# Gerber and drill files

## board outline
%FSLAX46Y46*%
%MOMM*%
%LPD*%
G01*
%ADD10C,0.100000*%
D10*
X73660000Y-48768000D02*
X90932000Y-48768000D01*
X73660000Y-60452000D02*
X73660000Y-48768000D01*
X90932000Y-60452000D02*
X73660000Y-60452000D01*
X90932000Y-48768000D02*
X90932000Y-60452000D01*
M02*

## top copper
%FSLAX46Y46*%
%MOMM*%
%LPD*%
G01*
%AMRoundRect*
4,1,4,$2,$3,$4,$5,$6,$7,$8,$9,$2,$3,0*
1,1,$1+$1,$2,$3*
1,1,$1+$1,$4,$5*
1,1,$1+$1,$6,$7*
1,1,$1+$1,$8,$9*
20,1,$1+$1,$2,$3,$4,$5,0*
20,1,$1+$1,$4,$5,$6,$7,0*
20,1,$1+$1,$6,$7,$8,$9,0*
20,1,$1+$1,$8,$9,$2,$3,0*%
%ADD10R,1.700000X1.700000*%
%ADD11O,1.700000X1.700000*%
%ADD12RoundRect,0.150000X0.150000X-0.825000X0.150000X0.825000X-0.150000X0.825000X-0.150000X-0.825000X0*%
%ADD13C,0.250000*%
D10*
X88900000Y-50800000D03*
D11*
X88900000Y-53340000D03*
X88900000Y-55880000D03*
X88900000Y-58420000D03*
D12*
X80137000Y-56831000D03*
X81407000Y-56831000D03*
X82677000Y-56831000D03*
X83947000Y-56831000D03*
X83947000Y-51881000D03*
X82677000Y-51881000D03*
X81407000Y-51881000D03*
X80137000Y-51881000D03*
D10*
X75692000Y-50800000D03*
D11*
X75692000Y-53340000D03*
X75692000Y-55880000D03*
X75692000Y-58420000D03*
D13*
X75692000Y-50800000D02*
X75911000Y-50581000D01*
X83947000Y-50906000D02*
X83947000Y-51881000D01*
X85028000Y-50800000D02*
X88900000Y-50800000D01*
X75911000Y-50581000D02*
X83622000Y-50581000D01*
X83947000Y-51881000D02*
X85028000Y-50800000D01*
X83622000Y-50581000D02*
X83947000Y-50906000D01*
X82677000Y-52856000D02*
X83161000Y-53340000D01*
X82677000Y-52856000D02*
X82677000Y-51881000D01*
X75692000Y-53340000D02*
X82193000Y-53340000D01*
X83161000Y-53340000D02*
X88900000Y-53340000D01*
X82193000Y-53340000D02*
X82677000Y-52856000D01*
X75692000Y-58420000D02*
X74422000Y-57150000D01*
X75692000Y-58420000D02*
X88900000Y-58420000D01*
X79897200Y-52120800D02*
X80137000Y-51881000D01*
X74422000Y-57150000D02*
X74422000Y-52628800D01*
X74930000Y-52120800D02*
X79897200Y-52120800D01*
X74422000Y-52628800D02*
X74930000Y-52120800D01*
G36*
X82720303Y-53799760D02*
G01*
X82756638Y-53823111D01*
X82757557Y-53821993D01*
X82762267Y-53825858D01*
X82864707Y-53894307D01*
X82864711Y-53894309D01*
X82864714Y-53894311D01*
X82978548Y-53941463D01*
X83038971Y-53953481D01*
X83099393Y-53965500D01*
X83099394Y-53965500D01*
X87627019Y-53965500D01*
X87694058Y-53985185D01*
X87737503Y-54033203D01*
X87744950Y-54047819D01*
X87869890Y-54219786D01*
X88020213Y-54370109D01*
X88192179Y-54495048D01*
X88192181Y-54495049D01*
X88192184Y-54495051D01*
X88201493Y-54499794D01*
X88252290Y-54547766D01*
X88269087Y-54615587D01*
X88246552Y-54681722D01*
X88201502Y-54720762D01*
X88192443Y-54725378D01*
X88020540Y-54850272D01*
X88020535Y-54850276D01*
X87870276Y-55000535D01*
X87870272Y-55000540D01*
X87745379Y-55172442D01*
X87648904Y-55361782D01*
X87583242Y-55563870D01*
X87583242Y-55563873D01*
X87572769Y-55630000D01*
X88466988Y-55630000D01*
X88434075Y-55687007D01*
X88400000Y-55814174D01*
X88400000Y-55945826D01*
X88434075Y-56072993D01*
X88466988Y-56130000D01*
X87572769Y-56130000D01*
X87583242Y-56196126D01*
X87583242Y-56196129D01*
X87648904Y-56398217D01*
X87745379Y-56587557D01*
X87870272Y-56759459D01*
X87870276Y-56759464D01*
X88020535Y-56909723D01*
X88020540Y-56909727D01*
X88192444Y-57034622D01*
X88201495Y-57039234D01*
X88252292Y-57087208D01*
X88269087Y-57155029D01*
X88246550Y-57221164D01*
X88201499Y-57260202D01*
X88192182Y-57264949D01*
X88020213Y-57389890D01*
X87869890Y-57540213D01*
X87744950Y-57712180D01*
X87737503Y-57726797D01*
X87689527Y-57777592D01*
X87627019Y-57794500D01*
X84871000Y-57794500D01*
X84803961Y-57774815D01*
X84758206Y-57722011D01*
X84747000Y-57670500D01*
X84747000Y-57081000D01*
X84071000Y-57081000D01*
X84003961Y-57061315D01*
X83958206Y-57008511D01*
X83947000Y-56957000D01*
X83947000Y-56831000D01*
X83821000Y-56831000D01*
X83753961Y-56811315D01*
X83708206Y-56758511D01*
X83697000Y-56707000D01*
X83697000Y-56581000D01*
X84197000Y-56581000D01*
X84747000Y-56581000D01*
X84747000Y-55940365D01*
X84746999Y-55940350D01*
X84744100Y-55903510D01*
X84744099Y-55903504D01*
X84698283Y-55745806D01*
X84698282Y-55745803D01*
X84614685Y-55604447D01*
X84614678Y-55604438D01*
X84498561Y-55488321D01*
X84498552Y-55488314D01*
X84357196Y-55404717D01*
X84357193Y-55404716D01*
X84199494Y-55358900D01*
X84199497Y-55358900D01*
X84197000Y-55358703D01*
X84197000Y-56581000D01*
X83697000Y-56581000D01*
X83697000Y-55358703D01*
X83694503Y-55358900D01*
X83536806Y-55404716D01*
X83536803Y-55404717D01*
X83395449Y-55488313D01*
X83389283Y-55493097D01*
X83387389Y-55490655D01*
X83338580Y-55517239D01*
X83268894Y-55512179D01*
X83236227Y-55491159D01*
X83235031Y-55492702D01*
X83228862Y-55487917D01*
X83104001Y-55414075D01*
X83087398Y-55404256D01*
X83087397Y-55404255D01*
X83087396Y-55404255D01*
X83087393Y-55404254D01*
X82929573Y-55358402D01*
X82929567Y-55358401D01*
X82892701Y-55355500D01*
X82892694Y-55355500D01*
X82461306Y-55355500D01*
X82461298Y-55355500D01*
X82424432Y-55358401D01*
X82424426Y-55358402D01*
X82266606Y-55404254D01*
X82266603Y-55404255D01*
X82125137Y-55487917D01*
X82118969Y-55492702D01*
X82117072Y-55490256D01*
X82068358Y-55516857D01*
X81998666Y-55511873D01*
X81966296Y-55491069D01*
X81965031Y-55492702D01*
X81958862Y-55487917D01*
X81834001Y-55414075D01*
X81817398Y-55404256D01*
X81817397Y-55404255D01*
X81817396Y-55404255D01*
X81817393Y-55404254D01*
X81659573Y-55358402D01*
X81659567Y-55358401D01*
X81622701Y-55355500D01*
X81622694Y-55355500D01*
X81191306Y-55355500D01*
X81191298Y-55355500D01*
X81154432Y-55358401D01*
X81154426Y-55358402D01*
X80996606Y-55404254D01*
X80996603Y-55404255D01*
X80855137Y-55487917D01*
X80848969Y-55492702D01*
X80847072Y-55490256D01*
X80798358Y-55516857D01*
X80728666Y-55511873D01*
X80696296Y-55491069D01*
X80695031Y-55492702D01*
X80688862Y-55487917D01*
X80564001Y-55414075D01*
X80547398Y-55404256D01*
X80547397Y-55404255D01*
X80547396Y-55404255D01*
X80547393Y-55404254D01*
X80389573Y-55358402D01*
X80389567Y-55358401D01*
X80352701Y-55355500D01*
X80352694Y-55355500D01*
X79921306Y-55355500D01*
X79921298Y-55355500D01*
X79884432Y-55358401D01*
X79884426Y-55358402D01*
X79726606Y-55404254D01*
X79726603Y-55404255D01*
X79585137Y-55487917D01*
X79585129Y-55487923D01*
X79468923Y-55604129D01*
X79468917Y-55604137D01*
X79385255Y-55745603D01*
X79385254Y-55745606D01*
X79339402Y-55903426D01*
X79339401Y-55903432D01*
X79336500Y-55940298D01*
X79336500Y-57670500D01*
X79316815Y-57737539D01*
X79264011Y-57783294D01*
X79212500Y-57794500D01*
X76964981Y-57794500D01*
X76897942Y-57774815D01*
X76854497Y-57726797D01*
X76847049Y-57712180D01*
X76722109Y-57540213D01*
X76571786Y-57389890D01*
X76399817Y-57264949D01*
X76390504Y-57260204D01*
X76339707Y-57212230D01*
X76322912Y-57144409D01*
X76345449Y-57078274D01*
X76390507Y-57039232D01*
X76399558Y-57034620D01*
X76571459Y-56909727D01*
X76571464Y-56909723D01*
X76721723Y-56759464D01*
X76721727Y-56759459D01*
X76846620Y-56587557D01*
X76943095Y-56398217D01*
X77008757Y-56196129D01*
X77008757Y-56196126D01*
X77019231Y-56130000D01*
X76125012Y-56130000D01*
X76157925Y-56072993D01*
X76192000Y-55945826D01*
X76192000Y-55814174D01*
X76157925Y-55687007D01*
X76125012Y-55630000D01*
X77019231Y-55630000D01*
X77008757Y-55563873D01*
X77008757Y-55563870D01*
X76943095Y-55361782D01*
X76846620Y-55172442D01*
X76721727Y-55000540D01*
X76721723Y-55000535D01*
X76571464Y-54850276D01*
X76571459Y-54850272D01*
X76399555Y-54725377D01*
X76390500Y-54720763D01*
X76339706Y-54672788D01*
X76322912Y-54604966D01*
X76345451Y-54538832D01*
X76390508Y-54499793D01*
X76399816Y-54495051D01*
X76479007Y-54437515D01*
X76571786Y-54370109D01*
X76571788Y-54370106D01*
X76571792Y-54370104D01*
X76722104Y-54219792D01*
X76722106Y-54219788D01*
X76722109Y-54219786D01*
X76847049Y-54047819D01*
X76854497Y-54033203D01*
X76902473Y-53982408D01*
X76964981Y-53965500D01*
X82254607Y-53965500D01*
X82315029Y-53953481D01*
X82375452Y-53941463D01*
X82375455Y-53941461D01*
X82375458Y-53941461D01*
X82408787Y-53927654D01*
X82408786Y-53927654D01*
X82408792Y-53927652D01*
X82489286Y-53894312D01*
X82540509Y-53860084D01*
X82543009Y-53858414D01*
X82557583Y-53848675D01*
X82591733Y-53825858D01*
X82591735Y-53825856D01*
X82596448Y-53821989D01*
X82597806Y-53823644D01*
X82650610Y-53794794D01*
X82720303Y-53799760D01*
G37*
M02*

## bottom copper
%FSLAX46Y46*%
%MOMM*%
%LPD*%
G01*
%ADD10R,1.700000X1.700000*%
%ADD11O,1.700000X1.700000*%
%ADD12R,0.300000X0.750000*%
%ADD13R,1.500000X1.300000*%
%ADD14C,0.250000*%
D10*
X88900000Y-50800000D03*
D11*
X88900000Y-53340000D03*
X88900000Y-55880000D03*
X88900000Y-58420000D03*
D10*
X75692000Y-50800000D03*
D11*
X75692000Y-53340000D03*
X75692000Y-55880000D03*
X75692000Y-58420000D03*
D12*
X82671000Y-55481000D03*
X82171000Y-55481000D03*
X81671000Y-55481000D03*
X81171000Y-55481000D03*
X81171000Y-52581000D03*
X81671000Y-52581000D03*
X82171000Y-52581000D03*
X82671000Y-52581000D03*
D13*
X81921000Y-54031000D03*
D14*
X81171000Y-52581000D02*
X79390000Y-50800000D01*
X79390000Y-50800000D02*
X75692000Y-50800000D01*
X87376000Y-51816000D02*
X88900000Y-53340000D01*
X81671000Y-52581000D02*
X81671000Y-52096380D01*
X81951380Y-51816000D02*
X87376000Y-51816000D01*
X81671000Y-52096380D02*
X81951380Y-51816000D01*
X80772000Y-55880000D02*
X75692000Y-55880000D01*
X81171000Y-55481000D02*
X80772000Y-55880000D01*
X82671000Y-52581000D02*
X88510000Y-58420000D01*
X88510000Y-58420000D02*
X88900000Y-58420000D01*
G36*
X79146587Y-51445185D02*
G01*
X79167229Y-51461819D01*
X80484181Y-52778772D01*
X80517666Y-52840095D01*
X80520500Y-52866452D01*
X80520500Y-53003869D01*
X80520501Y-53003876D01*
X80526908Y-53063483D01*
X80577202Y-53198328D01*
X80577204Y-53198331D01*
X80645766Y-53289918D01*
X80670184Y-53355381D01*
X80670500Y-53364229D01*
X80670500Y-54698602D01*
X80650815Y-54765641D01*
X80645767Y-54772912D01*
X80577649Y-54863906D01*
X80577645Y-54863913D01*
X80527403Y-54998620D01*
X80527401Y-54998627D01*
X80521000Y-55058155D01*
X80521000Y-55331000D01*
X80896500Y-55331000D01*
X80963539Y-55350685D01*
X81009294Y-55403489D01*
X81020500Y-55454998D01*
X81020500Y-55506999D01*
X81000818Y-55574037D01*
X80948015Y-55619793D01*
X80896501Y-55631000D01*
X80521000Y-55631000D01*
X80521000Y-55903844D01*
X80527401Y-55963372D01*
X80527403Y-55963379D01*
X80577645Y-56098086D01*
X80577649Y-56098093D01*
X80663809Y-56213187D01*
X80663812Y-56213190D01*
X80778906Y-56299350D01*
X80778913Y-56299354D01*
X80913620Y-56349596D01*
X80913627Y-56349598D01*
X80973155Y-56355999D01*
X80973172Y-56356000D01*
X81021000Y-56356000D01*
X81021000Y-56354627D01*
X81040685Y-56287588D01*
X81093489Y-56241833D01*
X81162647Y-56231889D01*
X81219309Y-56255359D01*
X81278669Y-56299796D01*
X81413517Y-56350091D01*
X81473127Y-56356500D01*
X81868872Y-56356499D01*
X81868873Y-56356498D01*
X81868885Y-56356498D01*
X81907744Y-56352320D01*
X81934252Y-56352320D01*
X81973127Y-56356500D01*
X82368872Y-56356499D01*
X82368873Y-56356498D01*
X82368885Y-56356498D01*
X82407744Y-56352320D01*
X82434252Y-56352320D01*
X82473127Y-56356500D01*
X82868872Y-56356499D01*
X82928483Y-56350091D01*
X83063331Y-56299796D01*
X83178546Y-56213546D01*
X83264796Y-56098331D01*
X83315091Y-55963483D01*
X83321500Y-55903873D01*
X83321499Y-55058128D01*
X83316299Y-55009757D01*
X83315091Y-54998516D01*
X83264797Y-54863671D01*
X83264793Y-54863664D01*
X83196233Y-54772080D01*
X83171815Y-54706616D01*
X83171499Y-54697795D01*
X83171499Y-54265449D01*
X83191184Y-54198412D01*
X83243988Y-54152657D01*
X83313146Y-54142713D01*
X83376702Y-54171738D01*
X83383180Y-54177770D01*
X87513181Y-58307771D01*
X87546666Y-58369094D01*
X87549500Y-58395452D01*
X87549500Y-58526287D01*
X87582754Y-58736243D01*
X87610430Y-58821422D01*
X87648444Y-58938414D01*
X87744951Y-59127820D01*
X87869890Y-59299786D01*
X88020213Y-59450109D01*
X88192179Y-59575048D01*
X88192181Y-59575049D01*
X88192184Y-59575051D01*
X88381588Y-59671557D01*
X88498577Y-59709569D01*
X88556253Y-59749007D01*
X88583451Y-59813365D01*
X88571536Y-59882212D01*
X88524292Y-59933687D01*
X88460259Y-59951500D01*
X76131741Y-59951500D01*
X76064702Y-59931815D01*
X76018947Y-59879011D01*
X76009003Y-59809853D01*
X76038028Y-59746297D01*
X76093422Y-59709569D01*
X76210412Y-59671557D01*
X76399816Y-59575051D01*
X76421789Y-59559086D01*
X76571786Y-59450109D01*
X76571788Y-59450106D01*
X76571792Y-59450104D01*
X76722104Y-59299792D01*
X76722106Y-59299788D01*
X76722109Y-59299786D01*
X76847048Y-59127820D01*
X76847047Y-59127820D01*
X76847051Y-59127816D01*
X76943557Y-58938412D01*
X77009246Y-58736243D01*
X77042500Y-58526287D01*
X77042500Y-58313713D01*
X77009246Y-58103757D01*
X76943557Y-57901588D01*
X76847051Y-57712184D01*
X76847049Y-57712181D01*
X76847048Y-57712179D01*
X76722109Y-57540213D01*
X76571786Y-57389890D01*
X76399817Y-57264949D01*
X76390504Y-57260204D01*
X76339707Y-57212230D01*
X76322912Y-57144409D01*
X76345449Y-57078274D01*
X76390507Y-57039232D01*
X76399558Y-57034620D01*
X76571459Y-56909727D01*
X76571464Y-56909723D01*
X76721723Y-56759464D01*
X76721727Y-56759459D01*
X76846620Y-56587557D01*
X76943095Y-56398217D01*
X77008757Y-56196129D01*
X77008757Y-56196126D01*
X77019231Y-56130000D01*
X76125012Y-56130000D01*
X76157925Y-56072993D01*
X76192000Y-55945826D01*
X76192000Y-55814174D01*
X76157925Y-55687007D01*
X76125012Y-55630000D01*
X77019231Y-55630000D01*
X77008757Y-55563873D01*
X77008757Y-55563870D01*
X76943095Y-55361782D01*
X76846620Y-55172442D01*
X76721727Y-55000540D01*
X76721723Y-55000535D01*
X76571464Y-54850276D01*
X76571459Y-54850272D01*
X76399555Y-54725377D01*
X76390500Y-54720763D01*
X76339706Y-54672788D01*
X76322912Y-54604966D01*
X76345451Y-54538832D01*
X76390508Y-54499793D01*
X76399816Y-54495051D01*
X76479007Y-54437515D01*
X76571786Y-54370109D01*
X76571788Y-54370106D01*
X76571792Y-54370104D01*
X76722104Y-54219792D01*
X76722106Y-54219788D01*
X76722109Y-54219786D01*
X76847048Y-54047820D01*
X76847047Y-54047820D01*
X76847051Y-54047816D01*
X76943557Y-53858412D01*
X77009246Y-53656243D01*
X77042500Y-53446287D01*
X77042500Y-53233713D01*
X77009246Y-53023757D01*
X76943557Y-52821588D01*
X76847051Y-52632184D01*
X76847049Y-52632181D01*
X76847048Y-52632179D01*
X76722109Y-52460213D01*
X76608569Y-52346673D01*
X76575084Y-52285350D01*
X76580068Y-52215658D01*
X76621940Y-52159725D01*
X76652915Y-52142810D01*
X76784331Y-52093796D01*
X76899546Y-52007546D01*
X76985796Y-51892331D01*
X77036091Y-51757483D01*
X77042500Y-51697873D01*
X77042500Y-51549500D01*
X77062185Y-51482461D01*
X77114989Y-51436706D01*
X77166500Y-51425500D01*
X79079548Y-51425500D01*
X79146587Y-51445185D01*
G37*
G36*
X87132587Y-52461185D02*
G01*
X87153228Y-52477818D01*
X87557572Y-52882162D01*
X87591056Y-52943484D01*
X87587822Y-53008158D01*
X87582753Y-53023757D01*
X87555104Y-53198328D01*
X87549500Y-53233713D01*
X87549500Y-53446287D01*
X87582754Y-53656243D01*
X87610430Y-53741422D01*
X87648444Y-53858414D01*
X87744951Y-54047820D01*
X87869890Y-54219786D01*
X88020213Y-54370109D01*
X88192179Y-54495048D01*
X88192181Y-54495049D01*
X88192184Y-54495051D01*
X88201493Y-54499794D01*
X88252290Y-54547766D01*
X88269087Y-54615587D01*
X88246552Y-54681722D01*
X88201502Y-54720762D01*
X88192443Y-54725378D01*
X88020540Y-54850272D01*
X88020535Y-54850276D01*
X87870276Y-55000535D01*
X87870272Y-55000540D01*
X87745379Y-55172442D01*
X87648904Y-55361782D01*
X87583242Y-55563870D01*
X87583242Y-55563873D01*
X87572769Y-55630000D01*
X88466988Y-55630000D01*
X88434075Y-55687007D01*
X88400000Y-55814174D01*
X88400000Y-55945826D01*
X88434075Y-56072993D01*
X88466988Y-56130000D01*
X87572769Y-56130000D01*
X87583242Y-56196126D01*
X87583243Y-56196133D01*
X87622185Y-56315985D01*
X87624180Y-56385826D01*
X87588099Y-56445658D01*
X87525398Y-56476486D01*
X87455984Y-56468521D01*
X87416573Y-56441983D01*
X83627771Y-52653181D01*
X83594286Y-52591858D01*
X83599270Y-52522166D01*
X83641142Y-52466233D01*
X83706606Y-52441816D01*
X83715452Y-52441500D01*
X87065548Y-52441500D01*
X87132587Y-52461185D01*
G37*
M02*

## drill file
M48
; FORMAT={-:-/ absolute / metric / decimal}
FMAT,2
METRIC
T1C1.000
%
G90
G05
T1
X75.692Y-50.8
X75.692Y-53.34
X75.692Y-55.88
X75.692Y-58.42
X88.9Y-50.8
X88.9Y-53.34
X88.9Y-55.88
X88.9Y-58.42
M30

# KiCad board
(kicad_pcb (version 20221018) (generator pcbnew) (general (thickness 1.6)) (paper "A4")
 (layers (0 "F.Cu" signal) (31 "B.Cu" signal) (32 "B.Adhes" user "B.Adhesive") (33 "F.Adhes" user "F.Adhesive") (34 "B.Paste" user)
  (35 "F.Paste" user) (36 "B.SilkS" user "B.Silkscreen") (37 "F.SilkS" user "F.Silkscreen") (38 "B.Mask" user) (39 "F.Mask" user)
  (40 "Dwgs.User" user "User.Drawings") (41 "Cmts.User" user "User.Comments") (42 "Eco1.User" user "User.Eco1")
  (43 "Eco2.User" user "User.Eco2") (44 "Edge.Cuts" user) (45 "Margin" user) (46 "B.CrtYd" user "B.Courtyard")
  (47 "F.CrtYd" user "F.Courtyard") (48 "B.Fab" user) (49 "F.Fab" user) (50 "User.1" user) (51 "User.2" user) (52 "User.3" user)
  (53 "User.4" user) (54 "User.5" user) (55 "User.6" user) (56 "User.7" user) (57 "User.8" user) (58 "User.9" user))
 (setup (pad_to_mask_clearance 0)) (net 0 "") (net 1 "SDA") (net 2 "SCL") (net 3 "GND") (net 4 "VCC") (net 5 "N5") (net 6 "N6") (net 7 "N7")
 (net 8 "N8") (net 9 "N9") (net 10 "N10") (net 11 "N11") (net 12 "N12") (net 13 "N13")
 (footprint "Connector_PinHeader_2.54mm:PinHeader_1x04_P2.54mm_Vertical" (layer "F.Cu") (at 88.9 50.8)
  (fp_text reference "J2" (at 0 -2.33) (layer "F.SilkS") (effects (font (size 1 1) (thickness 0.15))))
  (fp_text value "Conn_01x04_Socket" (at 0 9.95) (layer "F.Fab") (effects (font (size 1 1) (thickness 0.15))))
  (pad "1" thru_hole rect (at 0 0) (size 1.7 1.7) (drill 1) (layers "*.Cu" "*.Mask") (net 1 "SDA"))
  (pad "2" thru_hole oval (at 0 2.54) (size 1.7 1.7) (drill 1) (layers "*.Cu" "*.Mask") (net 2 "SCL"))
  (pad "3" thru_hole oval (at 0 5.08) (size 1.7 1.7) (drill 1) (layers "*.Cu" "*.Mask") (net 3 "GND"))
  (pad "4" thru_hole oval (at 0 7.62) (size 1.7 1.7) (drill 1) (layers "*.Cu" "*.Mask") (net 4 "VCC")))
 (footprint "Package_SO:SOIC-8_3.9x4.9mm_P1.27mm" (layer "F.Cu") (at 82.042 54.356 90)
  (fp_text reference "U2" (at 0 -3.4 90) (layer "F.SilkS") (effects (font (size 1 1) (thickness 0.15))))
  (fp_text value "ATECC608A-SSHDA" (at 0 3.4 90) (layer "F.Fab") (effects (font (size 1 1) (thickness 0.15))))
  (pad "1" smd roundrect (at -2.475 -1.905 90) (size 1.95 0.6) (layers "F.Cu" "F.Paste" "F.Mask") (roundrect_rratio 0.25) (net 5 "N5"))
  (pad "2" smd roundrect (at -2.475 -0.635 90) (size 1.95 0.6) (layers "F.Cu" "F.Paste" "F.Mask") (roundrect_rratio 0.25) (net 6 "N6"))
  (pad "3" smd roundrect (at -2.475 0.635 90) (size 1.95 0.6) (layers "F.Cu" "F.Paste" "F.Mask") (roundrect_rratio 0.25) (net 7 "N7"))
  (pad "4" smd roundrect (at -2.475 1.905 90) (size 1.95 0.6) (layers "F.Cu" "F.Paste" "F.Mask") (roundrect_rratio 0.25) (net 3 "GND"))
  (pad "5" smd roundrect (at 2.475 1.905 90) (size 1.95 0.6) (layers "F.Cu" "F.Paste" "F.Mask") (roundrect_rratio 0.25) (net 1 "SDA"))
  (pad "6" smd roundrect (at 2.475 0.635 90) (size 1.95 0.6) (layers "F.Cu" "F.Paste" "F.Mask") (roundrect_rratio 0.25) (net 2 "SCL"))
  (pad "7" smd roundrect (at 2.475 -0.635 90) (size 1.95 0.6) (layers "F.Cu" "F.Paste" "F.Mask") (roundrect_rratio 0.25) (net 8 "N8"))
  (pad "8" smd roundrect (at 2.475 -1.905 90) (size 1.95 0.6) (layers "F.Cu" "F.Paste" "F.Mask") (roundrect_rratio 0.25) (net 4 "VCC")))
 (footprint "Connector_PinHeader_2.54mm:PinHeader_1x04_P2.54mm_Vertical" (layer "F.Cu") (at 75.692 50.8)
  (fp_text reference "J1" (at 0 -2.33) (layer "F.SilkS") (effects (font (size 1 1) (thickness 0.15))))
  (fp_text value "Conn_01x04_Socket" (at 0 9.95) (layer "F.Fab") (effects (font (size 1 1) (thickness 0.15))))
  (pad "1" thru_hole rect (at 0 0) (size 1.7 1.7) (drill 1) (layers "*.Cu" "*.Mask") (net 1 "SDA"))
  (pad "2" thru_hole oval (at 0 2.54) (size 1.7 1.7) (drill 1) (layers "*.Cu" "*.Mask") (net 2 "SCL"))
  (pad "3" thru_hole oval (at 0 5.08) (size 1.7 1.7) (drill 1) (layers "*.Cu" "*.Mask") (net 3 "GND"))
  (pad "4" thru_hole oval (at 0 7.62) (size 1.7 1.7) (drill 1) (layers "*.Cu" "*.Mask") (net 4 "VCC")))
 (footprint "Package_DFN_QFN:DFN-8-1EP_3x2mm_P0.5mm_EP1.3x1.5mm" (layer "B.Cu") (at 81.921 54.031 90)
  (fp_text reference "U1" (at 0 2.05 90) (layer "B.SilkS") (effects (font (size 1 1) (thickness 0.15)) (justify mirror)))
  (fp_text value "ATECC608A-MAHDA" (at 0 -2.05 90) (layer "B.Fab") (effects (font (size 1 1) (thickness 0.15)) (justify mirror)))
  (pad "" smd rect (at -0.325 -0.375 90) (size 0.5 0.6) (layers "B.Paste"))
  (pad "" smd rect (at -0.325 0.375 90) (size 0.5 0.6) (layers "B.Paste"))
  (pad "" smd rect (at 0.325 -0.375 90) (size 0.5 0.6) (layers "B.Paste"))
  (pad "" smd rect (at 0.325 0.375 90) (size 0.5 0.6) (layers "B.Paste"))
  (pad "1" smd rect (at -1.45 0.75 90) (size 0.75 0.3) (layers "B.Cu" "B.Paste" "B.Mask") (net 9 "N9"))
  (pad "2" smd rect (at -1.45 0.25 90) (size 0.75 0.3) (layers "B.Cu" "B.Paste" "B.Mask") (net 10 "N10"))
  (pad "3" smd rect (at -1.45 -0.25 90) (size 0.75 0.3) (layers "B.Cu" "B.Paste" "B.Mask") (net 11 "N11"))
  (pad "4" smd rect (at -1.45 -0.75 90) (size 0.75 0.3) (layers "B.Cu" "B.Paste" "B.Mask") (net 3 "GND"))
  (pad "5" smd rect (at 1.45 -0.75 90) (size 0.75 0.3) (layers "B.Cu" "B.Paste" "B.Mask") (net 1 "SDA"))
  (pad "6" smd rect (at 1.45 -0.25 90) (size 0.75 0.3) (layers "B.Cu" "B.Paste" "B.Mask") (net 2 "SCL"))
  (pad "7" smd rect (at 1.45 0.25 90) (size 0.75 0.3) (layers "B.Cu" "B.Paste" "B.Mask") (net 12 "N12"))
  (pad "8" smd rect (at 1.45 0.75 90) (size 0.75 0.3) (layers "B.Cu" "B.Paste" "B.Mask") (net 4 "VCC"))
  (pad "9" smd rect (at 0 0 90) (size 1.3 1.5) (layers "B.Cu" "B.Mask") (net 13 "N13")))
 (gr_line (start 73.66 48.768) (end 90.932 48.768) (stroke (width 0.1) (type default)) (layer "Edge.Cuts"))
 (gr_line (start 73.66 60.452) (end 73.66 48.768) (stroke (width 0.1) (type default)) (layer "Edge.Cuts"))
 (gr_line (start 90.932 60.452) (end 73.66 60.452) (stroke (width 0.1) (type default)) (layer "Edge.Cuts"))
 (gr_line (start 90.932 48.768) (end 90.932 60.452) (stroke (width 0.1) (type default)) (layer "Edge.Cuts"))
 (segment (start 75.692 50.8) (end 75.911 50.581) (width 0.25) (layer "F.Cu") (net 1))
 (segment (start 83.947 50.906) (end 83.947 51.881) (width 0.25) (layer "F.Cu") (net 1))
 (segment (start 85.028 50.8) (end 88.9 50.8) (width 0.25) (layer "F.Cu") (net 1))
 (segment (start 75.911 50.581) (end 83.622 50.581) (width 0.25) (layer "F.Cu") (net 1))
 (segment (start 83.947 51.881) (end 85.028 50.8) (width 0.25) (layer "F.Cu") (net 1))
 (segment (start 83.622 50.581) (end 83.947 50.906) (width 0.25) (layer "F.Cu") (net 1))
 (segment (start 81.171 52.581) (end 79.39 50.8) (width 0.25) (layer "B.Cu") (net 1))
 (segment (start 79.39 50.8) (end 75.692 50.8) (width 0.25) (layer "B.Cu") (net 1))
 (segment (start 82.677 52.856) (end 83.161 53.34) (width 0.25) (layer "F.Cu") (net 2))
 (segment (start 82.677 52.856) (end 82.677 51.881) (width 0.25) (layer "F.Cu") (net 2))
 (segment (start 75.692 53.34) (end 82.193 53.34) (width 0.25) (layer "F.Cu") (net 2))
 (segment (start 83.161 53.34) (end 88.9 53.34) (width 0.25) (layer "F.Cu") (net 2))
 (segment (start 82.193 53.34) (end 82.677 52.856) (width 0.25) (layer "F.Cu") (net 2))
 (segment (start 87.376 51.816) (end 88.9 53.34) (width 0.25) (layer "B.Cu") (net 2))
 (segment (start 81.671 52.581) (end 81.671 52.09638) (width 0.25) (layer "B.Cu") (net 2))
 (segment (start 81.95138 51.816) (end 87.376 51.816) (width 0.25) (layer "B.Cu") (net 2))
 (segment (start 81.671 52.09638) (end 81.95138 51.816) (width 0.25) (layer "B.Cu") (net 2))
 (segment (start 80.772 55.88) (end 75.692 55.88) (width 0.25) (layer "B.Cu") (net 3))
 (segment (start 81.171 55.481) (end 80.772 55.88) (width 0.25) (layer "B.Cu") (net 3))
 (segment (start 75.692 58.42) (end 74.422 57.15) (width 0.25) (layer "F.Cu") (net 4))
 (segment (start 75.692 58.42) (end 88.9 58.42) (width 0.25) (layer "F.Cu") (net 4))
 (segment (start 79.8972 52.1208) (end 80.137 51.881) (width 0.25) (layer "F.Cu") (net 4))
 (segment (start 74.422 57.15) (end 74.422 52.6288) (width 0.25) (layer "F.Cu") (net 4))
 (segment (start 74.93 52.1208) (end 79.8972 52.1208) (width 0.25) (layer "F.Cu") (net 4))
 (segment (start 74.422 52.6288) (end 74.93 52.1208) (width 0.25) (layer "F.Cu") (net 4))
 (segment (start 82.671 52.581) (end 88.51 58.42) (width 0.25) (layer "B.Cu") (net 4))
 (segment (start 88.51 58.42) (end 88.9 58.42) (width 0.25) (layer "B.Cu") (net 4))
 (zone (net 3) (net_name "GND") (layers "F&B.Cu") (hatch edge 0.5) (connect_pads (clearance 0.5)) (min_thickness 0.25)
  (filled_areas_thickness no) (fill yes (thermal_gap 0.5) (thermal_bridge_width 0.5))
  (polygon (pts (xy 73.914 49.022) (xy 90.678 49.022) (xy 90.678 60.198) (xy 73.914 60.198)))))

